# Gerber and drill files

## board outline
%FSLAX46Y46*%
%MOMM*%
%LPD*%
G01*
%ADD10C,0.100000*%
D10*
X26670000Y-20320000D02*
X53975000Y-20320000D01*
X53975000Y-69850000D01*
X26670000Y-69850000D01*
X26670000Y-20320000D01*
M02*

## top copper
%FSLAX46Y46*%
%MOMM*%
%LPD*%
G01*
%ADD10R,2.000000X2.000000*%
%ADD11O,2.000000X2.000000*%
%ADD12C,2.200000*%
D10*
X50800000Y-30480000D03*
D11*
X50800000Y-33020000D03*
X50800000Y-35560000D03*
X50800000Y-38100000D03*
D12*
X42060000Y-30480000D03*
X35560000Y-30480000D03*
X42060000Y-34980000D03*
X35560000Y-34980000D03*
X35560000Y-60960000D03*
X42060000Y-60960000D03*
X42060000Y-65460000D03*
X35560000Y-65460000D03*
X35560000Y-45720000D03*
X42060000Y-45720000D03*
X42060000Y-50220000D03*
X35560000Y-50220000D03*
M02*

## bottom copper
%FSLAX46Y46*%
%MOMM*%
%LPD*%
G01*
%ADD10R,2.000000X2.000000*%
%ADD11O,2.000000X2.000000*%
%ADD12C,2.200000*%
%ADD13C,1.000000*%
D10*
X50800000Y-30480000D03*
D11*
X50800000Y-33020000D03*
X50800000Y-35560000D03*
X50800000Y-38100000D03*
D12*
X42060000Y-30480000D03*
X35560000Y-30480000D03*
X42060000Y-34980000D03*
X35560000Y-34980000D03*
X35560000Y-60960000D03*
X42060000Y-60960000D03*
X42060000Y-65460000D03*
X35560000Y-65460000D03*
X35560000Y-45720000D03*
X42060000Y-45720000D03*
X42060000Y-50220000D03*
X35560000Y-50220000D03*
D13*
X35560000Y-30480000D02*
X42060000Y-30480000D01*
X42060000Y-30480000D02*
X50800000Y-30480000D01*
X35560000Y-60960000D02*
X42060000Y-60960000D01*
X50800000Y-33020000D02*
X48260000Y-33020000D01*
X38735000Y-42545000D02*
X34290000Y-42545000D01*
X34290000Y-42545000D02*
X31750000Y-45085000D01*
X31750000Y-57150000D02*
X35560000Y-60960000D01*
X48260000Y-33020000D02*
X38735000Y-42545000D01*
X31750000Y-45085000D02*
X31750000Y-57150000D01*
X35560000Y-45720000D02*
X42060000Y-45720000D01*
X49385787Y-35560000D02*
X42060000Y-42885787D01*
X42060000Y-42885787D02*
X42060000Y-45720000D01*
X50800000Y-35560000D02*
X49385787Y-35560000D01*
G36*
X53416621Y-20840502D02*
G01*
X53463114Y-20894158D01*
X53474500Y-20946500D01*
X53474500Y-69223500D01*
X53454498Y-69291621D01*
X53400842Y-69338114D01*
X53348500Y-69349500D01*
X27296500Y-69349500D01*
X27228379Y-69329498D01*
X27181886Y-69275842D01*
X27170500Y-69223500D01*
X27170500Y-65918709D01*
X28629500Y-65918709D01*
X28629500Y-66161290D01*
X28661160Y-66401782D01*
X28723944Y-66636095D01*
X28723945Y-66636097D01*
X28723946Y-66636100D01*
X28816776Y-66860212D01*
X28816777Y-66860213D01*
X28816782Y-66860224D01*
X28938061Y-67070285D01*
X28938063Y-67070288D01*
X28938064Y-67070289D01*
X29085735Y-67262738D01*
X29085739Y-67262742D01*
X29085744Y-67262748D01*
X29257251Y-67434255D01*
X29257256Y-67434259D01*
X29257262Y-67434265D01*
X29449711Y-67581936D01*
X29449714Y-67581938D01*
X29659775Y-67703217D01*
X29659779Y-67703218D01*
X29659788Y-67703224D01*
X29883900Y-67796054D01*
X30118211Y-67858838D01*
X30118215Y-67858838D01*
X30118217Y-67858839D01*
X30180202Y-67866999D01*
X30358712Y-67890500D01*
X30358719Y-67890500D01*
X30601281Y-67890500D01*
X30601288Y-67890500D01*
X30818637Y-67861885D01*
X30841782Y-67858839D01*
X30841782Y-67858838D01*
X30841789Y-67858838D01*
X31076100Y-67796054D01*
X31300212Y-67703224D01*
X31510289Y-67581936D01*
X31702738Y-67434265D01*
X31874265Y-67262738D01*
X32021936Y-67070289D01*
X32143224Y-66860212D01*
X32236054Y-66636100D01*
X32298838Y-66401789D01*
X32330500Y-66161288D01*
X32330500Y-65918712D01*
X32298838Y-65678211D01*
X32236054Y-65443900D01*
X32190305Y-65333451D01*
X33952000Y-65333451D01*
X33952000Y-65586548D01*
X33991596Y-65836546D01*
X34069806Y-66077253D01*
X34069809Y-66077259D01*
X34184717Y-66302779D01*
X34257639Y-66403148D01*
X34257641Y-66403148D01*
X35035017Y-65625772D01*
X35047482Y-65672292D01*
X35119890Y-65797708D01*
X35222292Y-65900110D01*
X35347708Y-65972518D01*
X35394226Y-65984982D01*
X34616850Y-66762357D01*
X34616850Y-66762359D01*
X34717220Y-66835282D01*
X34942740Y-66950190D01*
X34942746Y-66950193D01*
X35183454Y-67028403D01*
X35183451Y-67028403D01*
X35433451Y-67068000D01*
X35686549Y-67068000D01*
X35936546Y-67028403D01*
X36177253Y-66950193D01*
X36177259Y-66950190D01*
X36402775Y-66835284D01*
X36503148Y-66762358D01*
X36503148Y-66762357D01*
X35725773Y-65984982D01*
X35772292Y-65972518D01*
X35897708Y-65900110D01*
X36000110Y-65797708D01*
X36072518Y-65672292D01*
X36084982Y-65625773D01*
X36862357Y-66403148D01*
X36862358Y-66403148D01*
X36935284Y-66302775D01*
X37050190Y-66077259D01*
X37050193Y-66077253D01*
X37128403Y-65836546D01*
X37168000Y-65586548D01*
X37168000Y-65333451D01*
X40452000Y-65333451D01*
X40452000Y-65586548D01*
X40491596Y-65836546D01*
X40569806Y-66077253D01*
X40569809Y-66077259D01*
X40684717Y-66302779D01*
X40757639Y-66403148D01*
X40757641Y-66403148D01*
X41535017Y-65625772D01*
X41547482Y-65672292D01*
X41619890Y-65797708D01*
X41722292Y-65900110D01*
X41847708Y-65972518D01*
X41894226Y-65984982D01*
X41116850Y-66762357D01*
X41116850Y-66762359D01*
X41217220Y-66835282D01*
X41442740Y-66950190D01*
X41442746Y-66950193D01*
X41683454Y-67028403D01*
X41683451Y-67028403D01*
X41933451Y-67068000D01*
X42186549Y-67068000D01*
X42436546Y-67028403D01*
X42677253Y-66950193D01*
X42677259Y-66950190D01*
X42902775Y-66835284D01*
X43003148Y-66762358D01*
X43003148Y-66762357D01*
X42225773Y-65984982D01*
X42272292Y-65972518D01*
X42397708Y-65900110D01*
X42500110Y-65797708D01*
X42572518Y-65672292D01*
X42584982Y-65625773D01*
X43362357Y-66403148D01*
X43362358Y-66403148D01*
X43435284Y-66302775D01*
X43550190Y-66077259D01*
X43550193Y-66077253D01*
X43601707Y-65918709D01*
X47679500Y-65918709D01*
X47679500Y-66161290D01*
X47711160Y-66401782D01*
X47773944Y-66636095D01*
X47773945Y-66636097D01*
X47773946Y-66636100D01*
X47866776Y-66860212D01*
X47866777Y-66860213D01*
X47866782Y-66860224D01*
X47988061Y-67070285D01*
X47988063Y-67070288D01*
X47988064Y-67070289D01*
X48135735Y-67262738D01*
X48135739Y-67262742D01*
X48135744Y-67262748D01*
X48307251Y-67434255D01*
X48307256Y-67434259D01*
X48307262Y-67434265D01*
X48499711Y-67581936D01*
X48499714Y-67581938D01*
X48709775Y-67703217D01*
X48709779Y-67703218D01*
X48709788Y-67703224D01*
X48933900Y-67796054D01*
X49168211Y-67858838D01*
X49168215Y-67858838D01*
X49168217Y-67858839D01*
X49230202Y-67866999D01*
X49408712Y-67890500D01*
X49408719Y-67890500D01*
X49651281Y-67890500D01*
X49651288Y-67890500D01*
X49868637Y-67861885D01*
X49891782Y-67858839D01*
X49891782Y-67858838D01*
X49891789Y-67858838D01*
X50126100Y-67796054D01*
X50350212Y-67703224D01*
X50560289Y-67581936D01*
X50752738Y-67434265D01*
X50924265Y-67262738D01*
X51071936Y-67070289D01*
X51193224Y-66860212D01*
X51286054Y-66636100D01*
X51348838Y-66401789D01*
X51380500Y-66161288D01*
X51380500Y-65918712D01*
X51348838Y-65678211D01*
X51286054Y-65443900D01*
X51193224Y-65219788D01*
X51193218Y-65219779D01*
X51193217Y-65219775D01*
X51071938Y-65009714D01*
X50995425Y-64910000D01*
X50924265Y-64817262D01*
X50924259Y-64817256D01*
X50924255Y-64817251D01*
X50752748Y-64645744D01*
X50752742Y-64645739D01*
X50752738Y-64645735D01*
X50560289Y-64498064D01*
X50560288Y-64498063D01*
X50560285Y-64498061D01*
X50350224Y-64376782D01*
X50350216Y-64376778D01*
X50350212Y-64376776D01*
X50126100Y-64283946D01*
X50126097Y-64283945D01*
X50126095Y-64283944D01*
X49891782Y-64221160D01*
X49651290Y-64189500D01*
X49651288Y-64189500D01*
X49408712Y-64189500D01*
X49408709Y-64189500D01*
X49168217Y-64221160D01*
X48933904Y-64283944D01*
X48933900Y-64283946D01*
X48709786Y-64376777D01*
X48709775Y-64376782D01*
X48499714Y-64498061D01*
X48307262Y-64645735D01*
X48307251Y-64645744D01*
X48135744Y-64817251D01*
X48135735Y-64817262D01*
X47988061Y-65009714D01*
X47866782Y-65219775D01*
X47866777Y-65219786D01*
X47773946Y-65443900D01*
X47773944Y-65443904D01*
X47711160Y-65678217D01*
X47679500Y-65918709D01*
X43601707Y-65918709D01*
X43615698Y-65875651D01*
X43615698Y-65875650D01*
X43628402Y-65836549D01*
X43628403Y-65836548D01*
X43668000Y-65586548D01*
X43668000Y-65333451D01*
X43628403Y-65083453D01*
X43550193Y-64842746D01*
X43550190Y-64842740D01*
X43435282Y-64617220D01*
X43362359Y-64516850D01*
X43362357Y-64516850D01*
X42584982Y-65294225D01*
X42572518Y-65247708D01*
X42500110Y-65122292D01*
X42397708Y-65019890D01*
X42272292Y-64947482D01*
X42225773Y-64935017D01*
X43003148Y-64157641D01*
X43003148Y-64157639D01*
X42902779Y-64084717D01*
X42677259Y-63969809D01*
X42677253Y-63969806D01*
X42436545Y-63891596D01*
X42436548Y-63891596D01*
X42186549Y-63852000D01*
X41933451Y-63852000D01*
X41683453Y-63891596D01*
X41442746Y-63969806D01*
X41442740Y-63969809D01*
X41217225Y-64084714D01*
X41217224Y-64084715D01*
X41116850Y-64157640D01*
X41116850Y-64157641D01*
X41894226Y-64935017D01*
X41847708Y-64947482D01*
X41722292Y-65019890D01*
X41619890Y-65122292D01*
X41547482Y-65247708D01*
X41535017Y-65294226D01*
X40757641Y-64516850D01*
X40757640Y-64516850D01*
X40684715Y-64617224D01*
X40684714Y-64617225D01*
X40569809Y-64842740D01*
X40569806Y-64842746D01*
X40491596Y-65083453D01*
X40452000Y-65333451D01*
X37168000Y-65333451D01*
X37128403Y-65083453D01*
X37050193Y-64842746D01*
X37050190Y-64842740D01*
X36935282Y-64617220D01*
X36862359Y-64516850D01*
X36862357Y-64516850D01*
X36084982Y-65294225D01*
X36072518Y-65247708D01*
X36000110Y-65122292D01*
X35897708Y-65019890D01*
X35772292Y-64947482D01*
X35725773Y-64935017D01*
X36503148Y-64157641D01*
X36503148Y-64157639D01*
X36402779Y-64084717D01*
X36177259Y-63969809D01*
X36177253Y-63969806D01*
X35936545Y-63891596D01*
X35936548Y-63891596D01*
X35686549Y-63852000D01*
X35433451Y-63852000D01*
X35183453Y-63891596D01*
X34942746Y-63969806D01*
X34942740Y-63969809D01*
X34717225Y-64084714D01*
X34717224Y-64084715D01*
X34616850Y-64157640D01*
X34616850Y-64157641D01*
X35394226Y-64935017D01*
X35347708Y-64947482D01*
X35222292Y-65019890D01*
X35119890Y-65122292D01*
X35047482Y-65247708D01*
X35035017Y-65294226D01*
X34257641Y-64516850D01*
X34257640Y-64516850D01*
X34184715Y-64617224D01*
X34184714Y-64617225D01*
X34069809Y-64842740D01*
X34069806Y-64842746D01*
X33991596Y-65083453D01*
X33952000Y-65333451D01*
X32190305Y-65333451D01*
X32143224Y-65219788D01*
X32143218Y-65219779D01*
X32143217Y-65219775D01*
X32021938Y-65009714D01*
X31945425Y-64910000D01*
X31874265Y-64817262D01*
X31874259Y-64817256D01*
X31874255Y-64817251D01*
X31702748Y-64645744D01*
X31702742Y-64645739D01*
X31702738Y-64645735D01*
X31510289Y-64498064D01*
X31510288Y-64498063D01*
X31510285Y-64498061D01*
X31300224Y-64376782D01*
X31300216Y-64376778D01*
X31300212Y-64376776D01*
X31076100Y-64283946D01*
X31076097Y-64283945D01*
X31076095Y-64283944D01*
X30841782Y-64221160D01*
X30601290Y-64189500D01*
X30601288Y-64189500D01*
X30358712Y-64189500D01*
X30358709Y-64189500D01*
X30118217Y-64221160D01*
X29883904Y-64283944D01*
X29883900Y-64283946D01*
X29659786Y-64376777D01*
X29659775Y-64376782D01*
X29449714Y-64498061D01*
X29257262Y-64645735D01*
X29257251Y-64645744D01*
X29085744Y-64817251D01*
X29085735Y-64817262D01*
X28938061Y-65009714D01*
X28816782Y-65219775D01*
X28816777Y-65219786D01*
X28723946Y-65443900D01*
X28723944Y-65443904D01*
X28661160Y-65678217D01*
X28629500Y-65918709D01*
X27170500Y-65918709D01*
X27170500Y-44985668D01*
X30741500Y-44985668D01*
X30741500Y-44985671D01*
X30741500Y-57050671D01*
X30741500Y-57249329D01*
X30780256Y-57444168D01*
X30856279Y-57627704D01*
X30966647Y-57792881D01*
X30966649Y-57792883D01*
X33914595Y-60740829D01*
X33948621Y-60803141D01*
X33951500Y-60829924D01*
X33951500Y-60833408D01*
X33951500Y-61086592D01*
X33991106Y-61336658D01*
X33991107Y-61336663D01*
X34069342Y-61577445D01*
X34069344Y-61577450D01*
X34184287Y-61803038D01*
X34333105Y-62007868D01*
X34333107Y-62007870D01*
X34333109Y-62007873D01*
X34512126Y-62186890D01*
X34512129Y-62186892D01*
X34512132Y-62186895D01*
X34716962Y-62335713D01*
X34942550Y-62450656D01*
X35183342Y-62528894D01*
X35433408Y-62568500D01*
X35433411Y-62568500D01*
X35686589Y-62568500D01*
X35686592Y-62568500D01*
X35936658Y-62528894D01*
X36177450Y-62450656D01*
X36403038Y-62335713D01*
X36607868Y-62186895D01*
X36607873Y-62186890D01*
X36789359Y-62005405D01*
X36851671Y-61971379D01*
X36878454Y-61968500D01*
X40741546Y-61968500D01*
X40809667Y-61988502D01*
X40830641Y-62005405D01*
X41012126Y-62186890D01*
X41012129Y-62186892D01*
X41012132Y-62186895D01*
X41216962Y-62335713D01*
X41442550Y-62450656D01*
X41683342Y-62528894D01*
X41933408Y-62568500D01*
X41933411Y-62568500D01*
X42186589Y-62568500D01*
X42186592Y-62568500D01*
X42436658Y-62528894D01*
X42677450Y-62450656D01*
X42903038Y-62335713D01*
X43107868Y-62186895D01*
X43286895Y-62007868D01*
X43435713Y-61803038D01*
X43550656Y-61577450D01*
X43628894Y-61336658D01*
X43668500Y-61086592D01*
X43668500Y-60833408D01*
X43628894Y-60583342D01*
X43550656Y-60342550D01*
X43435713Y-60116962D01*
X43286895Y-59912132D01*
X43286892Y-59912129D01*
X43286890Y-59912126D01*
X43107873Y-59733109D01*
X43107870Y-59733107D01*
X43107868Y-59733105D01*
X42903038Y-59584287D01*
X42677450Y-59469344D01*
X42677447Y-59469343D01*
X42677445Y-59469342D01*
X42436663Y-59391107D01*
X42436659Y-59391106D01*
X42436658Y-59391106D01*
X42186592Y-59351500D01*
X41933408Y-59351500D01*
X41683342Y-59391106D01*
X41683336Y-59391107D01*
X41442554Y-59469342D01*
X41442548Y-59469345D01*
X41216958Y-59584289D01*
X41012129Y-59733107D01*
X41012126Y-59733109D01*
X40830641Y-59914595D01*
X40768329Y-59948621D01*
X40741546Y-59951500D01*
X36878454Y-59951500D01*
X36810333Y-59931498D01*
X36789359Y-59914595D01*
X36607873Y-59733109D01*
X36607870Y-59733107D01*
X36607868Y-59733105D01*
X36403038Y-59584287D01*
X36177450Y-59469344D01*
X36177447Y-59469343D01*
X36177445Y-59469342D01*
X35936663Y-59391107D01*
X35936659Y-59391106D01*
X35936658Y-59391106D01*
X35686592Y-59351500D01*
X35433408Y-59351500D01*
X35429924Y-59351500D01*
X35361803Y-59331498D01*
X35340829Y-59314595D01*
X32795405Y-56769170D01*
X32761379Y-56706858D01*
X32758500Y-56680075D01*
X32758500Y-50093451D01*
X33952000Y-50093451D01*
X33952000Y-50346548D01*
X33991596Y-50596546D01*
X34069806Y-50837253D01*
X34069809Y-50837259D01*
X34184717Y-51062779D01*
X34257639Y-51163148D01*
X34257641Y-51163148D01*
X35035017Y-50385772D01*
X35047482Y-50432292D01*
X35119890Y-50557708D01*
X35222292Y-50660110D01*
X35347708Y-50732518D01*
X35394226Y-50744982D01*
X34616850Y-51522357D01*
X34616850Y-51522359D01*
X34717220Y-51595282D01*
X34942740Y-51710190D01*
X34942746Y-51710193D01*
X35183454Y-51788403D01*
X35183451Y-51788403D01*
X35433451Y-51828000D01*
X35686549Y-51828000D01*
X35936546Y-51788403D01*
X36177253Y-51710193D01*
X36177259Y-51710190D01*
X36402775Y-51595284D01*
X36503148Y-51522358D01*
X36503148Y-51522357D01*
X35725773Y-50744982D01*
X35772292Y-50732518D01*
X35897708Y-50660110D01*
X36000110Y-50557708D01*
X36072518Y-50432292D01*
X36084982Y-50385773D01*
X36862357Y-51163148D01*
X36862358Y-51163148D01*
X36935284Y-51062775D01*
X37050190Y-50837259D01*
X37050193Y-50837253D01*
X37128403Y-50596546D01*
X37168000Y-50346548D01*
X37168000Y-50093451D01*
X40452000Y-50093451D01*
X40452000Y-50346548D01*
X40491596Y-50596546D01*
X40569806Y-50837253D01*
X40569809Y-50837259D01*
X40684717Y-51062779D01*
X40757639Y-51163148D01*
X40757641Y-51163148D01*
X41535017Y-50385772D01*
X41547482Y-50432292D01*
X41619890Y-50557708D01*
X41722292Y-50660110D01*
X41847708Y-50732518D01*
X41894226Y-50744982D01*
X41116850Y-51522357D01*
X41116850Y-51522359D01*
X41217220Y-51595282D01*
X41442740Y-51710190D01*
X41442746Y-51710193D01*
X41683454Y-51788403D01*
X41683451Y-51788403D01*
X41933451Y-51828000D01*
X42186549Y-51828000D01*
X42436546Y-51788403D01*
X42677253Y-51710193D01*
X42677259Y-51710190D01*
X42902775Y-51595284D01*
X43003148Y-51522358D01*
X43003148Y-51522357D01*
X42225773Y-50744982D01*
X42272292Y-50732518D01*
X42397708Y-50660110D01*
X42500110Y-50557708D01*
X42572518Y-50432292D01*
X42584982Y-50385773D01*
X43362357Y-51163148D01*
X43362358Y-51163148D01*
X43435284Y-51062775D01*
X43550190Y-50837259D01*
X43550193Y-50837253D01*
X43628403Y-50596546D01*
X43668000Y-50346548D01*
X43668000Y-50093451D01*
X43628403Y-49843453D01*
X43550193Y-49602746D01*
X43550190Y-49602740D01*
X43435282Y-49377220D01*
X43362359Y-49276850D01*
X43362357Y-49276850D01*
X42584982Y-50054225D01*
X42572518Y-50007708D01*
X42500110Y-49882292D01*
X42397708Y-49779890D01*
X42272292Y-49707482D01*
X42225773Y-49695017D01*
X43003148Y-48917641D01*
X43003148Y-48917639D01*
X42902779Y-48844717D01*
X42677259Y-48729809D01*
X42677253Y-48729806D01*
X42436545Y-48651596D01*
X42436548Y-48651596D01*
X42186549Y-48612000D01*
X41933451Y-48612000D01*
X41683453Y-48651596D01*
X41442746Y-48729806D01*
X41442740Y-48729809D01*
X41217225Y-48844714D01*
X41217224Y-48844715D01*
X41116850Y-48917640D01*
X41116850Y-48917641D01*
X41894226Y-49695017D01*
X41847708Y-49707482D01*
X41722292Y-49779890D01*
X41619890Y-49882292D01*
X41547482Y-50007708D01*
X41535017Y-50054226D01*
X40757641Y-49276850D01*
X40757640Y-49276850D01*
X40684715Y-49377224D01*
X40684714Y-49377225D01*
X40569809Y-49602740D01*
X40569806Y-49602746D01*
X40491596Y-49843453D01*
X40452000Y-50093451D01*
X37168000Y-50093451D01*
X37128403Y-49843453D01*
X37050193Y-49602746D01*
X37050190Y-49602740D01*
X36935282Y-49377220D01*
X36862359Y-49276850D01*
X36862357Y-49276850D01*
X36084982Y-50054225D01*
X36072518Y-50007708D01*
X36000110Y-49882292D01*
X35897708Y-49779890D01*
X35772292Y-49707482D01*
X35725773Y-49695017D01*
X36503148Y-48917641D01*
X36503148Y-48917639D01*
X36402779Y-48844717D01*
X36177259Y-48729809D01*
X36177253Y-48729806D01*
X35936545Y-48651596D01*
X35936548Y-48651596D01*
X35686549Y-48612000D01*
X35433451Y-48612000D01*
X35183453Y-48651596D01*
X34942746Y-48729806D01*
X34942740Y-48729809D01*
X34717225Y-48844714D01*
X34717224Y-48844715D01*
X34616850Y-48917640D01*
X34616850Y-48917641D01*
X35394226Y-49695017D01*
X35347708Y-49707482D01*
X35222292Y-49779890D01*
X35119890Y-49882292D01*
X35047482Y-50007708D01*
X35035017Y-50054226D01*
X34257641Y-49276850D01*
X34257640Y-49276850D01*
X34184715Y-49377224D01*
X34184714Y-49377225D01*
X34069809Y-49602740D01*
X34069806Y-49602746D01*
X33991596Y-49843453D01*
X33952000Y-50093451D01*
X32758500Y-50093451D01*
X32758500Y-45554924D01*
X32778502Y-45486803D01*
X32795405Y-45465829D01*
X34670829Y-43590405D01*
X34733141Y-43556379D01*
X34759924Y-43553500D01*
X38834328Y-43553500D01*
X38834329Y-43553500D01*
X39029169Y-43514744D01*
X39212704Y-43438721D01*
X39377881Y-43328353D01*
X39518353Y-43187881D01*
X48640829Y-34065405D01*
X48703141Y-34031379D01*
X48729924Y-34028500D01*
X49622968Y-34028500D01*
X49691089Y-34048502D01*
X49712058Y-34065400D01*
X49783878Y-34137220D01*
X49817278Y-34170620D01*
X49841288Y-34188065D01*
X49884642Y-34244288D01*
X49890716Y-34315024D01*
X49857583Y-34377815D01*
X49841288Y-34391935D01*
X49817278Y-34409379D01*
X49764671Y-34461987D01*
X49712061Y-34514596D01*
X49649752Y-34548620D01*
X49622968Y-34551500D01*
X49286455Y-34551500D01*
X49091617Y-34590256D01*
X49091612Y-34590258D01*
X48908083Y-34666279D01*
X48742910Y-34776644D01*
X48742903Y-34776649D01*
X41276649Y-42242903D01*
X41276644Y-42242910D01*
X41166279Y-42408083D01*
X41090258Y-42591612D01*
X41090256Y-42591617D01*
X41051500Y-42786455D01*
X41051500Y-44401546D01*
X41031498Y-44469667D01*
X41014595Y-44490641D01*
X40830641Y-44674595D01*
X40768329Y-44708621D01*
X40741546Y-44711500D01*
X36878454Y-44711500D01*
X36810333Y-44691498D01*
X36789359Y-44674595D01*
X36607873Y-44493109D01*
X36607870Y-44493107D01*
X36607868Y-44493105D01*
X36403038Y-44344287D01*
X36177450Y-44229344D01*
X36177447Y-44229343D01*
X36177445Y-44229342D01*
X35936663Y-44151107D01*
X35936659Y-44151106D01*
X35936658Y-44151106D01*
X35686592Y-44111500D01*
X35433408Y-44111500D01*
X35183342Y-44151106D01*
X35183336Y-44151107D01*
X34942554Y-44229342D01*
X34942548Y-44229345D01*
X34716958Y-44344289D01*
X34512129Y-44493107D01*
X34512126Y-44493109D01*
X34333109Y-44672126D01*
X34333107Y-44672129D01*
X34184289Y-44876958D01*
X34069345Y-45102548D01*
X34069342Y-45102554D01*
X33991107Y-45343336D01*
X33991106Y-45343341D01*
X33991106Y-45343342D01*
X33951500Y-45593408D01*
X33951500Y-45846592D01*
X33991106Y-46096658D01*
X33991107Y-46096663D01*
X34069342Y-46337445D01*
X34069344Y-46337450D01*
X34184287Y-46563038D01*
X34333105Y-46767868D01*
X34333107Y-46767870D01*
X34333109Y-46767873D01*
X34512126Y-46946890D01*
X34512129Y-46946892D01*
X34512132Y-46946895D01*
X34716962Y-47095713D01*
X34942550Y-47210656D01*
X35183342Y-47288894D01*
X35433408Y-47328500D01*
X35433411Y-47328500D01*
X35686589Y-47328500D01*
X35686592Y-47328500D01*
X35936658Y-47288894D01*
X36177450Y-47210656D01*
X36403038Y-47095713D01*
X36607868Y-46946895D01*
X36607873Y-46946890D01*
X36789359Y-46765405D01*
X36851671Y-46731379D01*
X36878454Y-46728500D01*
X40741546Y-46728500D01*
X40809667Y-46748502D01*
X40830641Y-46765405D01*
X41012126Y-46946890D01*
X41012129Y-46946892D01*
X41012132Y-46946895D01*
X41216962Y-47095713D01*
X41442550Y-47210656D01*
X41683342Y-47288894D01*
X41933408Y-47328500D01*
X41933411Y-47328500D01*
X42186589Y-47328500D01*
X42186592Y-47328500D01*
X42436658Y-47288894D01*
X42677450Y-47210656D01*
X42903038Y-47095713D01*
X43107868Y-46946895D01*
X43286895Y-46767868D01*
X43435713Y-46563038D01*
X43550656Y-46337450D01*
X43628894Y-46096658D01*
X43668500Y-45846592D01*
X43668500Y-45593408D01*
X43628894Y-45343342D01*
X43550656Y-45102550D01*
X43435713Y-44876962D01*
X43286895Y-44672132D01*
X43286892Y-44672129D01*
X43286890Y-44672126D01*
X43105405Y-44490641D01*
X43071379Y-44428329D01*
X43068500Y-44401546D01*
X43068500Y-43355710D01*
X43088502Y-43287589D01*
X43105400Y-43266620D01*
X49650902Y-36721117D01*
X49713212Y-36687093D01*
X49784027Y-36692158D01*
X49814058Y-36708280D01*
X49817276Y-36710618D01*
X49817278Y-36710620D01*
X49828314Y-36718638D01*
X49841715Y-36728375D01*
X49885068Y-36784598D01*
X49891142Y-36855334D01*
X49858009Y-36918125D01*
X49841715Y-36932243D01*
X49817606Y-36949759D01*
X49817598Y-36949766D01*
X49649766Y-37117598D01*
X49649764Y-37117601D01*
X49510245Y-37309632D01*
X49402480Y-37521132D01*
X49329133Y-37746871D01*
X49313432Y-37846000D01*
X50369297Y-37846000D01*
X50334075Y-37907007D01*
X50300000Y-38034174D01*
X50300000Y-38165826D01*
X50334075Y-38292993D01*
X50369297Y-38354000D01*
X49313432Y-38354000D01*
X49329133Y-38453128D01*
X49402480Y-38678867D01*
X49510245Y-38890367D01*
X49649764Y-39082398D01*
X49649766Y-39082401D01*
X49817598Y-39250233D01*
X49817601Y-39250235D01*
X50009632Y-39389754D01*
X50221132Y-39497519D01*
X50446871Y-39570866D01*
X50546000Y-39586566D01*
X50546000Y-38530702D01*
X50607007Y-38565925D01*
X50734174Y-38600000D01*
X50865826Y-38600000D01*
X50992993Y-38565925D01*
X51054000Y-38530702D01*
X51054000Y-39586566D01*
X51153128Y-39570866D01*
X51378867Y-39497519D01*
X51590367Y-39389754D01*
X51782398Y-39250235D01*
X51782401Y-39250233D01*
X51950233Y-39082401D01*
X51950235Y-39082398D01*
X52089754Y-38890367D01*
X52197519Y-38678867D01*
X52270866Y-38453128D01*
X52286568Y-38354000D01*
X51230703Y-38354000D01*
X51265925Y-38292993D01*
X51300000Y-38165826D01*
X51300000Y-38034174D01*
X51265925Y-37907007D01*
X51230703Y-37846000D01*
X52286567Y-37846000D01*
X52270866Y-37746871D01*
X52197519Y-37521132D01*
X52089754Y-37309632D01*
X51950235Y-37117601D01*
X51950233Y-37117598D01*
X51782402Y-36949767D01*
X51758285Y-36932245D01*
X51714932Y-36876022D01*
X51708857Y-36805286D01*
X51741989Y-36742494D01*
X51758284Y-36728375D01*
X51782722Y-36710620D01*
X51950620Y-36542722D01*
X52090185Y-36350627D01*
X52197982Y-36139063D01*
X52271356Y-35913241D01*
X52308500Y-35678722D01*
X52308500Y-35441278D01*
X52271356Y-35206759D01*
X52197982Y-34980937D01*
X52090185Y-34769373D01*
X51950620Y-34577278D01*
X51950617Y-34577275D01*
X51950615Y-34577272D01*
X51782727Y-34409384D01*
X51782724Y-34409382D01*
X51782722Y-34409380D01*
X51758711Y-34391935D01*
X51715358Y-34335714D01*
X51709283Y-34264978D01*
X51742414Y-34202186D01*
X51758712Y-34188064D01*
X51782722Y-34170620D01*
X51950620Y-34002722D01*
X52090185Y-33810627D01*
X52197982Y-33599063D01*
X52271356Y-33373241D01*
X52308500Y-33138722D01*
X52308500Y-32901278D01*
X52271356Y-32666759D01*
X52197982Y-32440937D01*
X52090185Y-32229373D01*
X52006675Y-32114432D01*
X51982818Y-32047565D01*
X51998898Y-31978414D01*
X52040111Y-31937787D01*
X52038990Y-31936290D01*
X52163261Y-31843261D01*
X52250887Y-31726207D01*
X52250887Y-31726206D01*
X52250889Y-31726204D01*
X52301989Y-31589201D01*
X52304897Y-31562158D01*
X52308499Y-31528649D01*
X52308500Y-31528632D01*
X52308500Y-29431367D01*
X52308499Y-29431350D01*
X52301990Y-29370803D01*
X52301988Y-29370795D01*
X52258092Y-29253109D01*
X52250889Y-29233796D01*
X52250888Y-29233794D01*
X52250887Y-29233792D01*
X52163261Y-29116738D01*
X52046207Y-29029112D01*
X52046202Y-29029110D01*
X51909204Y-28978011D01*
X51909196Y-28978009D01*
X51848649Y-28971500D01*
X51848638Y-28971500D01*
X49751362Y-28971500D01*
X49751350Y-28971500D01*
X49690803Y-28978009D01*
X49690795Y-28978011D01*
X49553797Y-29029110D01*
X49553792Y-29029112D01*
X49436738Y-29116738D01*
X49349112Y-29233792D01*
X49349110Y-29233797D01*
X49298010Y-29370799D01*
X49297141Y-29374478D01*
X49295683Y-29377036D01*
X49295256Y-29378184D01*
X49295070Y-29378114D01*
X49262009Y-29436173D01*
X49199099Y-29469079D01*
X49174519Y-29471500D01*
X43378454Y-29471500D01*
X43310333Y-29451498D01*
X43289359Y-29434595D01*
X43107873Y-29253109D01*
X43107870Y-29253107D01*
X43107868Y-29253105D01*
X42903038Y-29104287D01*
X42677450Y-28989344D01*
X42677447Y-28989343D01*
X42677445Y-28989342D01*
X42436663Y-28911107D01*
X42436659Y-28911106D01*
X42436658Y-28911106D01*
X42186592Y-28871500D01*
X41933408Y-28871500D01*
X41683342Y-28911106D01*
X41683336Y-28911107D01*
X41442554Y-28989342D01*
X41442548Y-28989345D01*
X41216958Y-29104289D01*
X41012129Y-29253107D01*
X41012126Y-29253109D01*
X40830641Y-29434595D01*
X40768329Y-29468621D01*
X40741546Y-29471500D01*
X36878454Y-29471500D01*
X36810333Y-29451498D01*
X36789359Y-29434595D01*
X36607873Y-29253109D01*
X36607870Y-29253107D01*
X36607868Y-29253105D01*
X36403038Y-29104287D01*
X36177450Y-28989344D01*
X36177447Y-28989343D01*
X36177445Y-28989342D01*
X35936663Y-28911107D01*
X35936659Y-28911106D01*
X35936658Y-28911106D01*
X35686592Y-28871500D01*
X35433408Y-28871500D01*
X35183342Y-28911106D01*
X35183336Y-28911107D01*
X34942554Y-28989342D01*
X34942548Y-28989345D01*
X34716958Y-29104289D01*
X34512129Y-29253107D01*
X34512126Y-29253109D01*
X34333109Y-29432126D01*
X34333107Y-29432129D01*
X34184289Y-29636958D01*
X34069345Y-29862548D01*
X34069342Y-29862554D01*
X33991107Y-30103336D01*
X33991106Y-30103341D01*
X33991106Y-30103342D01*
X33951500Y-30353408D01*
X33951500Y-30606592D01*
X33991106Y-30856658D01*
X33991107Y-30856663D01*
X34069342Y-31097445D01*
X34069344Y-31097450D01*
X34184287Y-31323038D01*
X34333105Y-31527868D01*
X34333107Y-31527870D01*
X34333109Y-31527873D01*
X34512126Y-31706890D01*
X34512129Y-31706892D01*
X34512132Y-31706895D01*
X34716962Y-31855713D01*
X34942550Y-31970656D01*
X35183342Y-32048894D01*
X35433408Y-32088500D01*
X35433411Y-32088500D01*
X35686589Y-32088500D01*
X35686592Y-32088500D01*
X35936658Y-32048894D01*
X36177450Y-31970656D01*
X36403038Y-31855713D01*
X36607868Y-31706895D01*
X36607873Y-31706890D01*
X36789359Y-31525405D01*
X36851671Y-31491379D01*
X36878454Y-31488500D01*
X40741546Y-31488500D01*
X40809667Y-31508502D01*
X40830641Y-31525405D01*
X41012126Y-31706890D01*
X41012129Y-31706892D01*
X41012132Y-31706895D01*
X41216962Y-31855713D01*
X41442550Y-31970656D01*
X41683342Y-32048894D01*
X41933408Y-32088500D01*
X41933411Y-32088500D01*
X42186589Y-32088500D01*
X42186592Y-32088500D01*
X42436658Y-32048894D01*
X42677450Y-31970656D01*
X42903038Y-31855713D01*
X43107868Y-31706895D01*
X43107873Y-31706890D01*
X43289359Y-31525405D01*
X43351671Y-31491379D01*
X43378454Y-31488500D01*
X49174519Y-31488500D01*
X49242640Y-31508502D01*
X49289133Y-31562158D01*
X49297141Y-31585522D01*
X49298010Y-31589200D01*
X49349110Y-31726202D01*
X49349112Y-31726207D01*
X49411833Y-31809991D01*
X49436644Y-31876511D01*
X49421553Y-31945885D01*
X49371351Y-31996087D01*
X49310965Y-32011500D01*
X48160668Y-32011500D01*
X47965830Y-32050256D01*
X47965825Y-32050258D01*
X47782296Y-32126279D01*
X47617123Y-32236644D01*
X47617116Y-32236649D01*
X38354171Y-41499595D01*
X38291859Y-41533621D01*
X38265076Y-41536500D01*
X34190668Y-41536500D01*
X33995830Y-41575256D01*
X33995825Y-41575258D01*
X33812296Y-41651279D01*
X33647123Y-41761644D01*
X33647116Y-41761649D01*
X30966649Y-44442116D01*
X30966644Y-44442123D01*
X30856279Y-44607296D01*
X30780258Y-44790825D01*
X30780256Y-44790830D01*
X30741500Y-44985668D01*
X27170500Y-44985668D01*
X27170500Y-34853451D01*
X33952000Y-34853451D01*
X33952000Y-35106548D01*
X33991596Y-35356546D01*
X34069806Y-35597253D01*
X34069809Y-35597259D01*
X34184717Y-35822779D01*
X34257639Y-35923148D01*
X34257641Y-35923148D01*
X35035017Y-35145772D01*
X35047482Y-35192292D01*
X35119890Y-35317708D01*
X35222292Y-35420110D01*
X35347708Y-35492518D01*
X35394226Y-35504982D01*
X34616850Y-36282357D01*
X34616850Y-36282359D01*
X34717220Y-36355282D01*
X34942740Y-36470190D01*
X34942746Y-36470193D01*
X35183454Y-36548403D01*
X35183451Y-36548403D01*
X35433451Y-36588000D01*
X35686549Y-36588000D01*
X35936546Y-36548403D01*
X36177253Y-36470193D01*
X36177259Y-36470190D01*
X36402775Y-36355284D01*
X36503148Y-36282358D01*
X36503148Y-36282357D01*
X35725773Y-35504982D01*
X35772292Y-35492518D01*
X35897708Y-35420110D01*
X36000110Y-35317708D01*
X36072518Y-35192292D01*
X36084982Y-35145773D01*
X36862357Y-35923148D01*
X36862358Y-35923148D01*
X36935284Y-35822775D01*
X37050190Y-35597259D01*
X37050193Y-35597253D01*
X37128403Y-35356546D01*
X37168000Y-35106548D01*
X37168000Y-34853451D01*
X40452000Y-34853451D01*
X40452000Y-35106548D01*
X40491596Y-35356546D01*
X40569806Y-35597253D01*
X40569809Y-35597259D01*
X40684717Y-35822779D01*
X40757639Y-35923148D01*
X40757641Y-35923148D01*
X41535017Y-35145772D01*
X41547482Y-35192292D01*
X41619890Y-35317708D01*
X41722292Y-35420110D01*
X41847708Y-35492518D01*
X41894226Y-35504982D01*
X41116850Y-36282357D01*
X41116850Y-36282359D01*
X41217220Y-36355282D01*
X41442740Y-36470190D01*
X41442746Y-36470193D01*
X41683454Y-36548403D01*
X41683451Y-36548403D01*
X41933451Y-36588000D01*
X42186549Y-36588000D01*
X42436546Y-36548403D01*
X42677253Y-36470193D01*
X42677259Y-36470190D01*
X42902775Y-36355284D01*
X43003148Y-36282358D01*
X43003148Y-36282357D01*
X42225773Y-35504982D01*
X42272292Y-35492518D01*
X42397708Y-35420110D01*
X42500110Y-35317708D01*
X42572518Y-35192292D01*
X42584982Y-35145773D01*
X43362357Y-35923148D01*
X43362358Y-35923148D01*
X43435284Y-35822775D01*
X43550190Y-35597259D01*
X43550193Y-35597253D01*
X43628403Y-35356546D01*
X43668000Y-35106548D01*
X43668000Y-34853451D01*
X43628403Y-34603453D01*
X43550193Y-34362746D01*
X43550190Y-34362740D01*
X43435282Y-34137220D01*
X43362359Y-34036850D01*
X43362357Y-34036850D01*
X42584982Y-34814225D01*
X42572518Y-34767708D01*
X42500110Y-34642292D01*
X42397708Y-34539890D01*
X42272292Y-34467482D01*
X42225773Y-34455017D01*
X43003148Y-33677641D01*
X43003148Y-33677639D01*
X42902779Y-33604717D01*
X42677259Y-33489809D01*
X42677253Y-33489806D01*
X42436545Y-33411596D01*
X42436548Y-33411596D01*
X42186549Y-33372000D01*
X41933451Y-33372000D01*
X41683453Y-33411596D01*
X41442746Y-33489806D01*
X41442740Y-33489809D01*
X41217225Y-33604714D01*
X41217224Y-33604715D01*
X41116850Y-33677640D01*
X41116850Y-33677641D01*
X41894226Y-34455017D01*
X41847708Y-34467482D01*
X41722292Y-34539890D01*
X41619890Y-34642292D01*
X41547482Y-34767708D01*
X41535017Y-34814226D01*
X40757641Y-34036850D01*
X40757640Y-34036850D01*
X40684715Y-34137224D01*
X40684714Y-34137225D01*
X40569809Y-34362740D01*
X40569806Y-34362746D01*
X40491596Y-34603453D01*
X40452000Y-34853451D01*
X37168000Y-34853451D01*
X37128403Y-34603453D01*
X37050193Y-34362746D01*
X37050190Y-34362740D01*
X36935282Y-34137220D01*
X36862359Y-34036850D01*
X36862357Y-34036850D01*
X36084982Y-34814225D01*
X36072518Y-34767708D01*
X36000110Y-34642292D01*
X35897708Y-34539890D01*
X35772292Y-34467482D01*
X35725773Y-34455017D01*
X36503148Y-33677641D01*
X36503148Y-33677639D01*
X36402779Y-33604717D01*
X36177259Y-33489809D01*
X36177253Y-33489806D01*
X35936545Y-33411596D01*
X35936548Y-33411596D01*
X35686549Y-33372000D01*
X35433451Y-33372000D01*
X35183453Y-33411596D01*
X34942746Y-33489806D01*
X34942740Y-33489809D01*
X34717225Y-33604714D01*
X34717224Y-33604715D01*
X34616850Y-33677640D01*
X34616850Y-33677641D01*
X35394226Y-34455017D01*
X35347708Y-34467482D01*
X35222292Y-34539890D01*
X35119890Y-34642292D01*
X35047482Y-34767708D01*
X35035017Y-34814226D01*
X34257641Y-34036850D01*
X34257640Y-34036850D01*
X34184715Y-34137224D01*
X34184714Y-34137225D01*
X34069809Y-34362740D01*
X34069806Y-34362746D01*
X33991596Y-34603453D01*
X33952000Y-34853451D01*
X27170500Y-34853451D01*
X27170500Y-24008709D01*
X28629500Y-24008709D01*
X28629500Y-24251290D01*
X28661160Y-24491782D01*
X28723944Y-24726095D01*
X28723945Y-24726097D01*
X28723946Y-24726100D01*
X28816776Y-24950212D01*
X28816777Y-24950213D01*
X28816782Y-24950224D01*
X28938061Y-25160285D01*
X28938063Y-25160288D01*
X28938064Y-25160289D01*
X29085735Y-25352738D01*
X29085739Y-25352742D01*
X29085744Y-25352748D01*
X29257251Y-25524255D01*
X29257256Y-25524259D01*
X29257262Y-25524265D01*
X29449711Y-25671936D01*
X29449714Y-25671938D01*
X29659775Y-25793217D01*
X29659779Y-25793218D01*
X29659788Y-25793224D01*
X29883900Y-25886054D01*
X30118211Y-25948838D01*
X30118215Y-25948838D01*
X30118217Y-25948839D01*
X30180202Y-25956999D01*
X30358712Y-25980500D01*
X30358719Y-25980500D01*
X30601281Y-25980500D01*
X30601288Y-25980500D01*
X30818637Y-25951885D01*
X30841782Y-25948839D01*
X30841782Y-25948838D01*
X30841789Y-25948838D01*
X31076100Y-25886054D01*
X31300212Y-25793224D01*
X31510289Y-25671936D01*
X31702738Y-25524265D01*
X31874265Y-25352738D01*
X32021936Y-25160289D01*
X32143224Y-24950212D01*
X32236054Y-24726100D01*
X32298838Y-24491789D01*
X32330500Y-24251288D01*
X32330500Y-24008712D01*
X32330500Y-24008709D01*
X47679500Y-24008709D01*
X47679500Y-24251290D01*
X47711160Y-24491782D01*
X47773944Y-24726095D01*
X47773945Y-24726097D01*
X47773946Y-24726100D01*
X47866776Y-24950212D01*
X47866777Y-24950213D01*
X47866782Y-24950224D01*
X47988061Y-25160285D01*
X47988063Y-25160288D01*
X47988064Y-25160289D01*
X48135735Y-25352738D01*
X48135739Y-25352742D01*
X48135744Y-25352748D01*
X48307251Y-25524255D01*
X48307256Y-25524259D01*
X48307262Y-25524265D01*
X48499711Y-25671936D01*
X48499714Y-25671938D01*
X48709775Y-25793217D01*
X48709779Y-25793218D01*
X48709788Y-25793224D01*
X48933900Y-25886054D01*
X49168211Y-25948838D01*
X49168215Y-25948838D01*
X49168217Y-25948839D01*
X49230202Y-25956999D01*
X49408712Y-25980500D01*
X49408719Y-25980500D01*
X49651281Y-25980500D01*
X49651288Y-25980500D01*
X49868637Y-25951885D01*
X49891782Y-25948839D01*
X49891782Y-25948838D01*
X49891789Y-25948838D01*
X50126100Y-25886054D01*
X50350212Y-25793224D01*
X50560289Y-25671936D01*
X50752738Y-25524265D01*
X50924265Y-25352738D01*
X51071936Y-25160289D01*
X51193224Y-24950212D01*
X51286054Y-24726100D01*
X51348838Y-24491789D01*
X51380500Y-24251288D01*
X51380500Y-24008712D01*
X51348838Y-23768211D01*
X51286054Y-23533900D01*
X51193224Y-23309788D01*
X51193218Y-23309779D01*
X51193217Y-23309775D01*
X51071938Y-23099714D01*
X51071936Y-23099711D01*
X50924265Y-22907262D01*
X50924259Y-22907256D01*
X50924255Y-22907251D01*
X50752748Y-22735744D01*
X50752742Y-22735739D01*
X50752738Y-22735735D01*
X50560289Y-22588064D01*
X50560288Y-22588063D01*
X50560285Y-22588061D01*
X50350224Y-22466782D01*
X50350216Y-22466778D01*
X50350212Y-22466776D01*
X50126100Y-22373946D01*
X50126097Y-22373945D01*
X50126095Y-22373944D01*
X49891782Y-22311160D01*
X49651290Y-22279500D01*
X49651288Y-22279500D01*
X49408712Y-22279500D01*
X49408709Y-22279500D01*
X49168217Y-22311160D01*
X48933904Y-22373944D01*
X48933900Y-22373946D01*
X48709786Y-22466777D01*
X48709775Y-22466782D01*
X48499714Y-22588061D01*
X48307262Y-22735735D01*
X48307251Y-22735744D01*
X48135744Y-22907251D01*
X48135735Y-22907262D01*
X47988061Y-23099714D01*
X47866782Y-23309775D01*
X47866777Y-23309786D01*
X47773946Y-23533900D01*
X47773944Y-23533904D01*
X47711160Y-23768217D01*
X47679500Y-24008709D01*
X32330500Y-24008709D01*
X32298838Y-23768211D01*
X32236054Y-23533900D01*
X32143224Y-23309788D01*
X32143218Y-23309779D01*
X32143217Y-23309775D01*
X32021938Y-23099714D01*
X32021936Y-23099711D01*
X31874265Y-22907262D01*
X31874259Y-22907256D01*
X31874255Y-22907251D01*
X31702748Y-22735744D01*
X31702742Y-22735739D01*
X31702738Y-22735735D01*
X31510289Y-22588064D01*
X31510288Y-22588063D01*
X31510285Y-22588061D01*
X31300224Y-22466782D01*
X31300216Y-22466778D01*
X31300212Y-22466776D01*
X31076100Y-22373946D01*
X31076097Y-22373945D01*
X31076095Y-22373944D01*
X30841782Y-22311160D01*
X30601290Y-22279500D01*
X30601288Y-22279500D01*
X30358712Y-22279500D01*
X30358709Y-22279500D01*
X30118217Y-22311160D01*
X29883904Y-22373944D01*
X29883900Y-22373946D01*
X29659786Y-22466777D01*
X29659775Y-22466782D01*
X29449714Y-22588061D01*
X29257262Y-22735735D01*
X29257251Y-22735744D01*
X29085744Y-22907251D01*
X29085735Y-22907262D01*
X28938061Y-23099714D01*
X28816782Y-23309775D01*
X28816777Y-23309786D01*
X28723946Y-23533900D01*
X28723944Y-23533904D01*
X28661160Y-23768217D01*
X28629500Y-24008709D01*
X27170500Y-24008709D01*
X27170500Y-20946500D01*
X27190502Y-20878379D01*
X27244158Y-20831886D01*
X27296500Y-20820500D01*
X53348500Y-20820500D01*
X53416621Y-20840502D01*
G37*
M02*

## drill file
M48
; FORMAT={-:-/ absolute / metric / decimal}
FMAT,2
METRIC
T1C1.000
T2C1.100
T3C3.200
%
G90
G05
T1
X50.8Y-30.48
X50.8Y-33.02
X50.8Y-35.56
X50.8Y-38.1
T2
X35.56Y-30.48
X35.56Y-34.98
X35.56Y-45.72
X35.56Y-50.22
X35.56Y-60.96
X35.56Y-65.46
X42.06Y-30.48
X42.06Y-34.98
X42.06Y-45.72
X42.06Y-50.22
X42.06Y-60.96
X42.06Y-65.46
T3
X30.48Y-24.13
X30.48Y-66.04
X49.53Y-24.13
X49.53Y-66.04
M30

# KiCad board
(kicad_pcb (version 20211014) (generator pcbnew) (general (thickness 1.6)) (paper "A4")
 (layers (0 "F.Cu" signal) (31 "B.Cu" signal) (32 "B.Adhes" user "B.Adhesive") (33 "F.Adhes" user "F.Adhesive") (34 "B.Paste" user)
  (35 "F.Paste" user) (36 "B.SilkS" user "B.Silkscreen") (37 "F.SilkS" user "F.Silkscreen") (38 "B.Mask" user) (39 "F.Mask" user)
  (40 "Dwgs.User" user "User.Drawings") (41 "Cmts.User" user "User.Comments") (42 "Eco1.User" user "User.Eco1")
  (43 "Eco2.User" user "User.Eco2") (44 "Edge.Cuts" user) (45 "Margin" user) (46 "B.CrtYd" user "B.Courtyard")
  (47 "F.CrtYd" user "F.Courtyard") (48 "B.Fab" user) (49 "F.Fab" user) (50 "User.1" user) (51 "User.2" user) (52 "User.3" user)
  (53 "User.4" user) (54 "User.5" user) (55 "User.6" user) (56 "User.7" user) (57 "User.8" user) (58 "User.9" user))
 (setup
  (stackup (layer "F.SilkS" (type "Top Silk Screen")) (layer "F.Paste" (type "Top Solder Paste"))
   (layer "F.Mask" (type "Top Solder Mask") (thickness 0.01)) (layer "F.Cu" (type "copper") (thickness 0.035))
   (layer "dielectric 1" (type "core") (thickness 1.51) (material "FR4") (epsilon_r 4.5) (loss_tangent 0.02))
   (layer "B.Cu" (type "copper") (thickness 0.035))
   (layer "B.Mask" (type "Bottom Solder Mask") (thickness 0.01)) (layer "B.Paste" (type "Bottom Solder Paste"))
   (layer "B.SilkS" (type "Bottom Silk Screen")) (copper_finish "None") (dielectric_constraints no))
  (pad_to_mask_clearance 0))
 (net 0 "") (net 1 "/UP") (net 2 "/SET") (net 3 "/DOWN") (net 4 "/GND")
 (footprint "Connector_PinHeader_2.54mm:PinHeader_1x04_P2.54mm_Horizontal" (layer "F.Cu") (at 50.8 30.48)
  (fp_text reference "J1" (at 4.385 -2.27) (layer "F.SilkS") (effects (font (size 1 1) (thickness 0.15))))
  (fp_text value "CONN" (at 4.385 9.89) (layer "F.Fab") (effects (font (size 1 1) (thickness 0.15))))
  (pad "1" thru_hole rect (at 0 0) (size 2 2) (drill 1) (layers *.Cu *.Mask) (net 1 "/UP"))
  (pad "2" thru_hole oval (at 0 2.54) (size 2 2) (drill 1) (layers *.Cu *.Mask) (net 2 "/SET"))
  (pad "3" thru_hole oval (at 0 5.08) (size 2 2) (drill 1) (layers *.Cu *.Mask) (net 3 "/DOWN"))
  (pad "4" thru_hole oval (at 0 7.62) (size 2 2) (drill 1) (layers *.Cu *.Mask) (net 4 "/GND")))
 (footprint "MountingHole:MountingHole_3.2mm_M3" (layer "F.Cu") (at 30.48 66.04)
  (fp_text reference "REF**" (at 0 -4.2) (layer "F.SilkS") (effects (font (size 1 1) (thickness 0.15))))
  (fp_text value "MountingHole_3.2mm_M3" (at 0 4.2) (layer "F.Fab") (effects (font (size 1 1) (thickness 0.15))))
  (pad "" np_thru_hole circle (at 0 0) (size 3.2 3.2) (drill 3.2) (layers *.Cu *.Mask)))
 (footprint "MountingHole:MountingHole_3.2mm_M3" (layer "F.Cu") (at 49.53 66.04)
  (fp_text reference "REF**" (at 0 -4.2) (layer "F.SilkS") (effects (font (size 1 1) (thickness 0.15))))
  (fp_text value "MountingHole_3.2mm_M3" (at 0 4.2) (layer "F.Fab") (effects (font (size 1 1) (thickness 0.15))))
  (pad "" np_thru_hole circle (at 0 0) (size 3.2 3.2) (drill 3.2) (layers *.Cu *.Mask)))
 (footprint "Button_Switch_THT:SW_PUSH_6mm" (layer "F.Cu") (at 35.56 30.48)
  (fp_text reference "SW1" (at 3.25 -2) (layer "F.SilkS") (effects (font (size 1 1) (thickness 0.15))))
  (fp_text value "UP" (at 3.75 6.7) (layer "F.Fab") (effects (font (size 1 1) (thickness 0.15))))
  (pad "1" thru_hole circle (at 6.5 0 90) (size 2.2 2.2) (drill 1.1) (layers *.Cu *.Mask) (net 1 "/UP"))
  (pad "1" thru_hole circle (at 0 0 90) (size 2.2 2.2) (drill 1.1) (layers *.Cu *.Mask) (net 1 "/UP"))
  (pad "2" thru_hole circle (at 6.5 4.5 90) (size 2.2 2.2) (drill 1.1) (layers *.Cu *.Mask) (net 4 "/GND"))
  (pad "2" thru_hole circle (at 0 4.5 90) (size 2.2 2.2) (drill 1.1) (layers *.Cu *.Mask) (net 4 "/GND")))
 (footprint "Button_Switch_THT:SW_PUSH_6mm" (layer "F.Cu") (at 35.56 60.96)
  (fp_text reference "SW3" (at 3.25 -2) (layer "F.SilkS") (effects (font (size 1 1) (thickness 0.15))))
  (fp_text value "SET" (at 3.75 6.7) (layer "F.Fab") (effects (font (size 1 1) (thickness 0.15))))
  (pad "1" thru_hole circle (at 0 0 90) (size 2.2 2.2) (drill 1.1) (layers *.Cu *.Mask) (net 2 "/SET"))
  (pad "1" thru_hole circle (at 6.5 0 90) (size 2.2 2.2) (drill 1.1) (layers *.Cu *.Mask) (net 2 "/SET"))
  (pad "2" thru_hole circle (at 6.5 4.5 90) (size 2.2 2.2) (drill 1.1) (layers *.Cu *.Mask) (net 4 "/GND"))
  (pad "2" thru_hole circle (at 0 4.5 90) (size 2.2 2.2) (drill 1.1) (layers *.Cu *.Mask) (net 4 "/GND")))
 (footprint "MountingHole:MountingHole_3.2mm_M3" (layer "F.Cu") (at 30.48 24.13)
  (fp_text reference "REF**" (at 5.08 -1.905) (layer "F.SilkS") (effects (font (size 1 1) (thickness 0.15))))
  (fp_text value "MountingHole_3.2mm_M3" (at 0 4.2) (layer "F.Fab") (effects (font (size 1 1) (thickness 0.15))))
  (pad "" np_thru_hole circle (at 0 0) (size 3.2 3.2) (drill 3.2) (layers *.Cu *.Mask)))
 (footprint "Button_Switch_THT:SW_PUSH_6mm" (layer "F.Cu") (at 35.56 45.72)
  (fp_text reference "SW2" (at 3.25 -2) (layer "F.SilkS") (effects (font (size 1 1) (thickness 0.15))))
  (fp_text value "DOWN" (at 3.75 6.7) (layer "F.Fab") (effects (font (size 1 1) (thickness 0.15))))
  (pad "1" thru_hole circle (at 0 0 90) (size 2.2 2.2) (drill 1.1) (layers *.Cu *.Mask) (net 3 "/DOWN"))
  (pad "1" thru_hole circle (at 6.5 0 90) (size 2.2 2.2) (drill 1.1) (layers *.Cu *.Mask "Dwgs.User") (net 3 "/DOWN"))
  (pad "2" thru_hole circle (at 6.5 4.5 90) (size 2.2 2.2) (drill 1.1) (layers *.Cu *.Mask) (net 4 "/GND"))
  (pad "2" thru_hole circle (at 0 4.5 90) (size 2.2 2.2) (drill 1.1) (layers *.Cu *.Mask) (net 4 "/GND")))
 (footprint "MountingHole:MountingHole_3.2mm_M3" (layer "F.Cu") (at 49.53 24.13)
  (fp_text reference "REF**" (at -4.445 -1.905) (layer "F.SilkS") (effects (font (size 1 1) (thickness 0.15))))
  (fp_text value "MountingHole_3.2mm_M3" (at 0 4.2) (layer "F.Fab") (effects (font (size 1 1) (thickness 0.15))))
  (pad "" np_thru_hole circle (at 0 0) (size 3.2 3.2) (drill 3.2) (layers *.Cu *.Mask)))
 (gr_rect (start 26.67 20.32) (end 53.975 69.85) (layer "Edge.Cuts") (width 0.1) (fill none))
 (segment (start 35.56 30.48) (end 42.06 30.48) (width 1) (layer "B.Cu") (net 1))
 (segment (start 42.06 30.48) (end 50.8 30.48) (width 1) (layer "B.Cu") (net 1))
 (segment (start 35.56 60.96) (end 42.06 60.96) (width 1) (layer "B.Cu") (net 2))
 (segment (start 50.8 33.02) (end 48.26 33.02) (width 1) (layer "B.Cu") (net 2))
 (segment (start 38.735 42.545) (end 34.29 42.545) (width 1) (layer "B.Cu") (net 2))
 (segment (start 34.29 42.545) (end 31.75 45.085) (width 1) (layer "B.Cu") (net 2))
 (segment (start 31.75 57.15) (end 35.56 60.96) (width 1) (layer "B.Cu") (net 2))
 (segment (start 48.26 33.02) (end 38.735 42.545) (width 1) (layer "B.Cu") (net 2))
 (segment (start 31.75 45.085) (end 31.75 57.15) (width 1) (layer "B.Cu") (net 2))
 (segment (start 35.56 45.72) (end 42.06 45.72) (width 1) (layer "B.Cu") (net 3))
 (segment (start 49.385787 35.56) (end 42.06 42.885787) (width 1) (layer "B.Cu") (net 3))
 (segment (start 42.06 42.885787) (end 42.06 45.72) (width 1) (layer "B.Cu") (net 3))
 (segment (start 50.8 35.56) (end 49.385787 35.56) (width 1) (layer "B.Cu") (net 3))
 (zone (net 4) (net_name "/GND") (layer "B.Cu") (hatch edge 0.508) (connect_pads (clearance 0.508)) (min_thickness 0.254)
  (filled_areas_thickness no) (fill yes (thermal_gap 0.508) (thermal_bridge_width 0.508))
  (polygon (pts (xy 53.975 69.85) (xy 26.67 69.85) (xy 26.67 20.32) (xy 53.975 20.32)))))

